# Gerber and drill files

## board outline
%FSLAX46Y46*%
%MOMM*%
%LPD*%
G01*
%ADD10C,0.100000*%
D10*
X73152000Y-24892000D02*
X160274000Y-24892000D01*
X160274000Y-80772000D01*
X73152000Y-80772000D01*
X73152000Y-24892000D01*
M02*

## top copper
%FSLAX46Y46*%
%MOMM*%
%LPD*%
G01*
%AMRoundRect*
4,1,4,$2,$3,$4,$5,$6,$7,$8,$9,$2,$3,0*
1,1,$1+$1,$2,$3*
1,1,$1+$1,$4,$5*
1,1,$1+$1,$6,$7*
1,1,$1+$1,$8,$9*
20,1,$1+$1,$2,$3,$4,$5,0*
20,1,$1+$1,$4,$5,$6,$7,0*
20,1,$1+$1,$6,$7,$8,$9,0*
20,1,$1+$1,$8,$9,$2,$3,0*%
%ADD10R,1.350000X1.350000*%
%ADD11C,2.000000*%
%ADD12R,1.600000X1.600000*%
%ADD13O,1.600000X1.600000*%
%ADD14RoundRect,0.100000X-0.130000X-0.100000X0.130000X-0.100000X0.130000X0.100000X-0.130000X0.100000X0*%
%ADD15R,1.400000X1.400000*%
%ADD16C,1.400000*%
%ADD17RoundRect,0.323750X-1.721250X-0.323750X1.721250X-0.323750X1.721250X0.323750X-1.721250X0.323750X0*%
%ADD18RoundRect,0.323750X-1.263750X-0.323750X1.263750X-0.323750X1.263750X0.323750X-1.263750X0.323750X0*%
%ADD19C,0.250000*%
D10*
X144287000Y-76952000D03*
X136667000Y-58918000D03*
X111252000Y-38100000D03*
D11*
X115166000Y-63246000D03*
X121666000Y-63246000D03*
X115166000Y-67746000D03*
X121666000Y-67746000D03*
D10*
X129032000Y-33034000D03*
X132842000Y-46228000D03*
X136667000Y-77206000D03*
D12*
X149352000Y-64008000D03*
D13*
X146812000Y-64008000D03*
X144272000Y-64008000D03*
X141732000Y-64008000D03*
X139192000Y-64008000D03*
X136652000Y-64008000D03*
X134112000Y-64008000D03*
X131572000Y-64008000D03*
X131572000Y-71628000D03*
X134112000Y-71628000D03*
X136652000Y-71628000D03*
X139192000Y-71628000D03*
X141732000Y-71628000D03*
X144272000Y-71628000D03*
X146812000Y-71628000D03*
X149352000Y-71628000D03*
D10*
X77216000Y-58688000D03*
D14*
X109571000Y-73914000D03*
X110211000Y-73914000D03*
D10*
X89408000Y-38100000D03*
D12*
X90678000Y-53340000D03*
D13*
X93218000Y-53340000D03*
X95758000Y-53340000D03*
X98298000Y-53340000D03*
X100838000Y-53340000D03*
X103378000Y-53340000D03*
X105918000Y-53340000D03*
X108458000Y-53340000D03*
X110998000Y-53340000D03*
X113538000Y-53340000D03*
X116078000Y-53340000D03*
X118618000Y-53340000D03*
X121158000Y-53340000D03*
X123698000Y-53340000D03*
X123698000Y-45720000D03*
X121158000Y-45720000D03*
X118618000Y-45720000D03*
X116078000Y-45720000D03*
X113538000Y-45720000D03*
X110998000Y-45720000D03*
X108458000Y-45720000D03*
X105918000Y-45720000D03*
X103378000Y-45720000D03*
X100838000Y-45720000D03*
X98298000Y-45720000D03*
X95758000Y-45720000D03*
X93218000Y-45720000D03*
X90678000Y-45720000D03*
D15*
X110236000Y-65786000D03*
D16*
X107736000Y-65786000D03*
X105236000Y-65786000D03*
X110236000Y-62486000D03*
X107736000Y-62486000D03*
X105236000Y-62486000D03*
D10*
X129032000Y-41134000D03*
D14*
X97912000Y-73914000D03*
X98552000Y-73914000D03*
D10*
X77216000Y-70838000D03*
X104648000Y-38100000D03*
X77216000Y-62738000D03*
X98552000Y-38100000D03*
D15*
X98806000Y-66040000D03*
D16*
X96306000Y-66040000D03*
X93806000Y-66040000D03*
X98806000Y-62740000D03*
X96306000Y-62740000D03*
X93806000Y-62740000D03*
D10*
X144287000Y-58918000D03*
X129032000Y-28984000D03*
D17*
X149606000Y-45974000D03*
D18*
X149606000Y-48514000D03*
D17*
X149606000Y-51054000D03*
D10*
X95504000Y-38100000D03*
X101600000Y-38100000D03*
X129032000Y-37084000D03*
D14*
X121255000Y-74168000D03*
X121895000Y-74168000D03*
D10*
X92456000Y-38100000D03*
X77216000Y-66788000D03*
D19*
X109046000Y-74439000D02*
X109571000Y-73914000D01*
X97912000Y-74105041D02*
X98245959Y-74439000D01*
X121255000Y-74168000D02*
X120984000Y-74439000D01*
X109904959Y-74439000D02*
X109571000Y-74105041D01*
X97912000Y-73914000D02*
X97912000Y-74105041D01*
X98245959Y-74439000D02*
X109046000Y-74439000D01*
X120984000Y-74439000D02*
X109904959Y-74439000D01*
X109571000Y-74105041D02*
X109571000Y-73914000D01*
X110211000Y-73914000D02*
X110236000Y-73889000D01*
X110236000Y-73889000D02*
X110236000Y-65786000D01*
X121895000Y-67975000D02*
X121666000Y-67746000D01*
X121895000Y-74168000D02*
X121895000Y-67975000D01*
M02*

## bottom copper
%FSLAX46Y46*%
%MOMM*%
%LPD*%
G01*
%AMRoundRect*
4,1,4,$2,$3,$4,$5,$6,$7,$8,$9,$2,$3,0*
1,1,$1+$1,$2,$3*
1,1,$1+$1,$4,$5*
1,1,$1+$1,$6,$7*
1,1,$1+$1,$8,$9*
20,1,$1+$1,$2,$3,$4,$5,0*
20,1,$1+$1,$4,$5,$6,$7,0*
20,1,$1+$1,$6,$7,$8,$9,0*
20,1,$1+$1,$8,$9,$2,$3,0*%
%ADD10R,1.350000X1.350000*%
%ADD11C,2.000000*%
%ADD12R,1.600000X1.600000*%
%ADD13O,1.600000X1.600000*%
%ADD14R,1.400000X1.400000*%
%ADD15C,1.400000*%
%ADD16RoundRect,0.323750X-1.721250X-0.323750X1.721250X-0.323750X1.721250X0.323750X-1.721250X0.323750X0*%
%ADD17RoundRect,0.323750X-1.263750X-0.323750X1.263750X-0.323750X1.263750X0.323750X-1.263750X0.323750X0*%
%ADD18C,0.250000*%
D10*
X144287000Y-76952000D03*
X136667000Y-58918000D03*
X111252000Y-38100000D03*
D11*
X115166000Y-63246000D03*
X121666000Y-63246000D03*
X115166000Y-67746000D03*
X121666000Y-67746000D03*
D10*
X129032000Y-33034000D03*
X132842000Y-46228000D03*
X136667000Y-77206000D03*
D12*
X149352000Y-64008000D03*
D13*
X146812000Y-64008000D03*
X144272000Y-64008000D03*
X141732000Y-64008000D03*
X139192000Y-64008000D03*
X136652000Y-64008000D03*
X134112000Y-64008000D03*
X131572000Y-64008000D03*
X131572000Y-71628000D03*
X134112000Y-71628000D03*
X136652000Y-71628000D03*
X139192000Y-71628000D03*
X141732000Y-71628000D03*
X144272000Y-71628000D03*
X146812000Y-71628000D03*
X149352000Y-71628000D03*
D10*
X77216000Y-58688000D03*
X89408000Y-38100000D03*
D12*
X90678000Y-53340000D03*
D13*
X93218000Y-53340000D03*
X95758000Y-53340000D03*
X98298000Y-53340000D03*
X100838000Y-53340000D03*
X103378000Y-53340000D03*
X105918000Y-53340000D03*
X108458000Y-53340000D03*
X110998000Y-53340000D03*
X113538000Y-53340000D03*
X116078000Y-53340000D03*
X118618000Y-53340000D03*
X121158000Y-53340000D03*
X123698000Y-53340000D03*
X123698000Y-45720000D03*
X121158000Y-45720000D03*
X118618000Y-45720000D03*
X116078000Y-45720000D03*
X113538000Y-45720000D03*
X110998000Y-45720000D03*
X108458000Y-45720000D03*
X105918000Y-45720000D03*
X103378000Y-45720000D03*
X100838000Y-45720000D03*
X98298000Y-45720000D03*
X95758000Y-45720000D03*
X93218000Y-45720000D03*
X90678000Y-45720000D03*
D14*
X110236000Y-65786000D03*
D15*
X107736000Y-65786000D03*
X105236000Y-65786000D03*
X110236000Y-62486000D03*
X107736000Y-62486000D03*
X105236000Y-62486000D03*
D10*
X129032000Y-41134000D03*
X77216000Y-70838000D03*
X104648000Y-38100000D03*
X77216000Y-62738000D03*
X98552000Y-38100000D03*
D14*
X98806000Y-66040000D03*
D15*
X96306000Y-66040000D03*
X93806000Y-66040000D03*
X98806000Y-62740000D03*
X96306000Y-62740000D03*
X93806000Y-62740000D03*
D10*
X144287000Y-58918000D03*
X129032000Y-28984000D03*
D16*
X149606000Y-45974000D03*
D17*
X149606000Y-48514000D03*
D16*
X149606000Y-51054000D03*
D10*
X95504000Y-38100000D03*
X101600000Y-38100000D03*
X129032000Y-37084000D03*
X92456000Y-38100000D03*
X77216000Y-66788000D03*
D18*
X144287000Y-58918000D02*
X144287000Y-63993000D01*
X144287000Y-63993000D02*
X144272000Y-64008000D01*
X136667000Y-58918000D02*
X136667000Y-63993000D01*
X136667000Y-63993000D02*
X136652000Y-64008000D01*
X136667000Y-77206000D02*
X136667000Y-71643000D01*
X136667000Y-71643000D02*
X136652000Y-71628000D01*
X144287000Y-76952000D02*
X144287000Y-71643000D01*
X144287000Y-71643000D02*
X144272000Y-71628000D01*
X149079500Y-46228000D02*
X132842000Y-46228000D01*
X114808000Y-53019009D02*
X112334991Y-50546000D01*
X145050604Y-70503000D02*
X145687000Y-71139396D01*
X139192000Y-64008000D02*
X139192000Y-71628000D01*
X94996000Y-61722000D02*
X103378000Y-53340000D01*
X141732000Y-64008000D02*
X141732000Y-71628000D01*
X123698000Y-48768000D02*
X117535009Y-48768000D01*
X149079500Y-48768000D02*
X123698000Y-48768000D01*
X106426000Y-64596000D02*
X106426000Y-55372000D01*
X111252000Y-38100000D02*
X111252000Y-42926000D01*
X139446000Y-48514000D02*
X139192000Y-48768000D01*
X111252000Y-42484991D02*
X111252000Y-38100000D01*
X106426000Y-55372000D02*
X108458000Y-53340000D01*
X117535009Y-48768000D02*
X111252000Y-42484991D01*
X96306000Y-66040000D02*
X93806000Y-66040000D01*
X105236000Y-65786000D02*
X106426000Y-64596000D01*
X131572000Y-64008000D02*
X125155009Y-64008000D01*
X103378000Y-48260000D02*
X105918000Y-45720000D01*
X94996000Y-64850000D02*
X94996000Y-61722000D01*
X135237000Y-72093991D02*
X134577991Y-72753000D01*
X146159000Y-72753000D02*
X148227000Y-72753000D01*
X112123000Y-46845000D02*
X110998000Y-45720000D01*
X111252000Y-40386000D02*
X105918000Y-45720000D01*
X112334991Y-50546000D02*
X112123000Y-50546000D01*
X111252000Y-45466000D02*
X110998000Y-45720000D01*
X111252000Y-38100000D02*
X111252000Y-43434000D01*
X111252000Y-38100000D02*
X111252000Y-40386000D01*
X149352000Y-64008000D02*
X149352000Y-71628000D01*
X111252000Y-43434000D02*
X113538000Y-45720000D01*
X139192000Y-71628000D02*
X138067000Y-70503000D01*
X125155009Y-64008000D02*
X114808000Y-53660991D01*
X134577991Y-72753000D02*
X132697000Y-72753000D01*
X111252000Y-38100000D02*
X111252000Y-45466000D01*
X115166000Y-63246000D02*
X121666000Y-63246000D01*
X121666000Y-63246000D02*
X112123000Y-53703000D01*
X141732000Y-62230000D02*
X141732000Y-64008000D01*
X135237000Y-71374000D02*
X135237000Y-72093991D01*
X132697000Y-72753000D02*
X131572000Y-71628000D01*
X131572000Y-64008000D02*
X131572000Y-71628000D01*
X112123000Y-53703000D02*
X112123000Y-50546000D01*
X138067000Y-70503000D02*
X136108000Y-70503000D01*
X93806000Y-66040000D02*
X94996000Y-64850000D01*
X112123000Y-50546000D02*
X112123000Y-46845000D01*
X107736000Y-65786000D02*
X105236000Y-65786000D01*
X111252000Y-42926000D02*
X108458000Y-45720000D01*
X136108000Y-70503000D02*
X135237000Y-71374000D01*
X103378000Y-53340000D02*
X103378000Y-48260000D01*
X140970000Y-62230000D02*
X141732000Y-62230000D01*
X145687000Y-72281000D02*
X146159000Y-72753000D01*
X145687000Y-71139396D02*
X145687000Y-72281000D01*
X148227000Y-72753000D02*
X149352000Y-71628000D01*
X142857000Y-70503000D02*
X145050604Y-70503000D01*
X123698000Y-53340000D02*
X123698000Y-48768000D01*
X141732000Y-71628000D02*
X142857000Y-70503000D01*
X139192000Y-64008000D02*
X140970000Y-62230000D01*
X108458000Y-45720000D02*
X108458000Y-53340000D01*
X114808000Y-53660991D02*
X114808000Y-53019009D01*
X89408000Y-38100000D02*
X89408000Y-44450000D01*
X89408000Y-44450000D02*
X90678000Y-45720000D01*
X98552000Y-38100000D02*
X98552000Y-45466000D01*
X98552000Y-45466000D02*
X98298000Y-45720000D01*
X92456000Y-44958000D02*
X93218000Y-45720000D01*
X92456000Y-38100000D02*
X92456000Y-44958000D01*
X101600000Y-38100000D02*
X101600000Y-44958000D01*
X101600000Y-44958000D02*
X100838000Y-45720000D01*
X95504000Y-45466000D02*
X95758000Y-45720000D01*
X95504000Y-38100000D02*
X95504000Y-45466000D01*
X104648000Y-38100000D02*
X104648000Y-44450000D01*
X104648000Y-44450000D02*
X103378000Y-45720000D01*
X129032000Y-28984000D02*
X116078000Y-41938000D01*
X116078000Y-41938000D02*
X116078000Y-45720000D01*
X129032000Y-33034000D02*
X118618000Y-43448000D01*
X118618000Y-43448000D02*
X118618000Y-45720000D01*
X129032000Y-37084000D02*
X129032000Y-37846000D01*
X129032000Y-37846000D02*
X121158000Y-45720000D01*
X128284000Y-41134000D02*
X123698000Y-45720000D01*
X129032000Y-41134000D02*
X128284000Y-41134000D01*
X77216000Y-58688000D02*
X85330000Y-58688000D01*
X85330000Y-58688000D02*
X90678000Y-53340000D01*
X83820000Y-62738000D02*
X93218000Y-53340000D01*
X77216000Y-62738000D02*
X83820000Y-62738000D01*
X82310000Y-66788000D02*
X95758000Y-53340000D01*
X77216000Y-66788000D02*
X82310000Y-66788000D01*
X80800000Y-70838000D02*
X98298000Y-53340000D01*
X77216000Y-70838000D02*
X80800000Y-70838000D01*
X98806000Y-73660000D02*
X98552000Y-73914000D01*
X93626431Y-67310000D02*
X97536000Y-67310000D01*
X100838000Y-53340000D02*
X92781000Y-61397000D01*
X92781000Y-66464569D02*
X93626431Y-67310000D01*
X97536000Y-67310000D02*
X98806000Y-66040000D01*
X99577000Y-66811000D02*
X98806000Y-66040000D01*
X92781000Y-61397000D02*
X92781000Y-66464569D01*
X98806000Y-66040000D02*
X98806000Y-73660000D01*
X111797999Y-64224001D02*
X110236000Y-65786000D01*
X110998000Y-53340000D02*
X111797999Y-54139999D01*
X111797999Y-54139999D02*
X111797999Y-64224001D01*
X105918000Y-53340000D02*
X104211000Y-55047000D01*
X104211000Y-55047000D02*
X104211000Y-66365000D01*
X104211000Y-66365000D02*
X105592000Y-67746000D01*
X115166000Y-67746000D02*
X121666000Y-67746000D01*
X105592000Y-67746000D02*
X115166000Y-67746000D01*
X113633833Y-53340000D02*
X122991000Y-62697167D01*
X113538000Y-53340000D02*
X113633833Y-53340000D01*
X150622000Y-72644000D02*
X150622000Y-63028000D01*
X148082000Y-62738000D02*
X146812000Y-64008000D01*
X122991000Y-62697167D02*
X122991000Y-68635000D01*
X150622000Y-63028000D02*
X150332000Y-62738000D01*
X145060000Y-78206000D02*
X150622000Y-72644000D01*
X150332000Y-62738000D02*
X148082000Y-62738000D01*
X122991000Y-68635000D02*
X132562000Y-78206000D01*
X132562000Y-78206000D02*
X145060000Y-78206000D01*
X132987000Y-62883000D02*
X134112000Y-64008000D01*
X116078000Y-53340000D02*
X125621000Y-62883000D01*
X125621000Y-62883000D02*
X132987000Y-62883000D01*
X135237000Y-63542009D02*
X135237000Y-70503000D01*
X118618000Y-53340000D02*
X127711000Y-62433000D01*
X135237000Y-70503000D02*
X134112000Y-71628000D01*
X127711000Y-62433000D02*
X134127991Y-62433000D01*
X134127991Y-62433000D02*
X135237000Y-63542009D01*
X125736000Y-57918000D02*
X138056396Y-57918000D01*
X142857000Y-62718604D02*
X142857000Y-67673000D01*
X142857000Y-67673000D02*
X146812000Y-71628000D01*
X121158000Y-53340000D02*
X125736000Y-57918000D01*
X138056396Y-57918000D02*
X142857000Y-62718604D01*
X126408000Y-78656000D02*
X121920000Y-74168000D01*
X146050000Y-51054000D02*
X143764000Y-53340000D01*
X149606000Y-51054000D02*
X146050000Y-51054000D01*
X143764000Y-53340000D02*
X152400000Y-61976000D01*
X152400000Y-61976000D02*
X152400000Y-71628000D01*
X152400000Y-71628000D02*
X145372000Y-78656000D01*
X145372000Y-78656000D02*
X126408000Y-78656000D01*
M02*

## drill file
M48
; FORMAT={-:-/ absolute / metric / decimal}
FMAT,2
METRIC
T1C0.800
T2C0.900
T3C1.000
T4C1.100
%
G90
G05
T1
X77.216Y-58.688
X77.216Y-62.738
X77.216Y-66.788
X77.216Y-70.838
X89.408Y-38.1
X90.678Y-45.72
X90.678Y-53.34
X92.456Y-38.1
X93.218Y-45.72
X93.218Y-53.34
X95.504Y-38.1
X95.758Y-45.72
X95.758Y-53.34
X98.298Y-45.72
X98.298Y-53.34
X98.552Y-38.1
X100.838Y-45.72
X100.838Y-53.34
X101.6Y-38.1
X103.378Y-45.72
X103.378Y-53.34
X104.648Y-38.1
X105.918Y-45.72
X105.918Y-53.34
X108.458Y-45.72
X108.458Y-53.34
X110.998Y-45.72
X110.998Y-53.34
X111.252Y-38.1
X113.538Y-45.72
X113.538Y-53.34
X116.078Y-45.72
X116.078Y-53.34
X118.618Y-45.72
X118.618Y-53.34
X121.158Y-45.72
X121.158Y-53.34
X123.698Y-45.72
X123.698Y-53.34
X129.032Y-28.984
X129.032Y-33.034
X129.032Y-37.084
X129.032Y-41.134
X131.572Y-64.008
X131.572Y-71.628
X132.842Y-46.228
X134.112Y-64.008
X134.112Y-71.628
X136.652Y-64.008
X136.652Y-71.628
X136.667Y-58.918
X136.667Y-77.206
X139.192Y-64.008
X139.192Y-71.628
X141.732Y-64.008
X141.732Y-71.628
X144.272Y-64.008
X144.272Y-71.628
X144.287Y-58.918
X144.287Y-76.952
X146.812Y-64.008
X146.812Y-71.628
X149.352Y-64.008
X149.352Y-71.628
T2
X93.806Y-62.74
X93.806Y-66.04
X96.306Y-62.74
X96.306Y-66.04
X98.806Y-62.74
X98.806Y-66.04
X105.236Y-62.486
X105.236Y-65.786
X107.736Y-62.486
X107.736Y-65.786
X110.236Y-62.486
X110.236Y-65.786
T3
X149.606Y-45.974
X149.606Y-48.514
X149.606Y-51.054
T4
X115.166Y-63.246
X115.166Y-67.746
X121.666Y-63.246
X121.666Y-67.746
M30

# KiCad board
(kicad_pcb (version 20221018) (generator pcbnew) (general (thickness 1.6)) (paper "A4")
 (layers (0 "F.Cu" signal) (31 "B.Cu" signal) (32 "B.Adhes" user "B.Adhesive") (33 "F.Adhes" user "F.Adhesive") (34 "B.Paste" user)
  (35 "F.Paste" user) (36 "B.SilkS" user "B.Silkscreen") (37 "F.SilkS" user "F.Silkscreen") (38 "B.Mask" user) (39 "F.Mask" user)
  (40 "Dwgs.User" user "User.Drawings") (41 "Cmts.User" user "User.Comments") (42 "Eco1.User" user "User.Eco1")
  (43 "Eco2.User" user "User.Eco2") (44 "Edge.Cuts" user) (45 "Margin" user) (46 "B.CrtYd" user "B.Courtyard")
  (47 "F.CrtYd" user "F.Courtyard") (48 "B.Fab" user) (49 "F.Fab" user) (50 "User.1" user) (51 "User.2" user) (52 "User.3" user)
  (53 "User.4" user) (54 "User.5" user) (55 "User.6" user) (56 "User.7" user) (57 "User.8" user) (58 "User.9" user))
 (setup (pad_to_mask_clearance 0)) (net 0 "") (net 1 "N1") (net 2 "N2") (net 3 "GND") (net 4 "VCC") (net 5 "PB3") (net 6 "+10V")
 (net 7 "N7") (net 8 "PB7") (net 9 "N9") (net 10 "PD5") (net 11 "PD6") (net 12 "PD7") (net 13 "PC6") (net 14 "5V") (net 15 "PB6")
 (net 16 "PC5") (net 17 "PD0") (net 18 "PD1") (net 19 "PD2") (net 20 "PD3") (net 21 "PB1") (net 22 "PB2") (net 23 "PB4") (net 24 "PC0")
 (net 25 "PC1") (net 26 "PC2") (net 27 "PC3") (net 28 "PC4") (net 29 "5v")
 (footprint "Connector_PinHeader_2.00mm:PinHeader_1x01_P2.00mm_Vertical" (layer "F.Cu") (at 144.287 76.952)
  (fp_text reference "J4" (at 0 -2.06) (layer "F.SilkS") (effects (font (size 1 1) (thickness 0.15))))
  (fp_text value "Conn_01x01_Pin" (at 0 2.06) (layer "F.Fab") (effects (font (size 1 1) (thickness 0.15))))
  (pad "1" thru_hole rect (at 0 0) (size 1.35 1.35) (drill 0.8) (layers "*.Cu" "*.Mask") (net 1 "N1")))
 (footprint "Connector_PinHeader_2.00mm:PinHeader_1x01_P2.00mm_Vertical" (layer "F.Cu") (at 136.667 58.918)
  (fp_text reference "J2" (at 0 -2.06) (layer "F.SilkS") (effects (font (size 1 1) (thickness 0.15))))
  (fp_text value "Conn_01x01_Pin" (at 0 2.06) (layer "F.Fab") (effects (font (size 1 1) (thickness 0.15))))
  (pad "1" thru_hole rect (at 0 0) (size 1.35 1.35) (drill 0.8) (layers "*.Cu" "*.Mask") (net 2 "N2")))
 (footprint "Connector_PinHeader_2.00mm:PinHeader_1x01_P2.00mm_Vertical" (layer "F.Cu") (at 111.252 38.1)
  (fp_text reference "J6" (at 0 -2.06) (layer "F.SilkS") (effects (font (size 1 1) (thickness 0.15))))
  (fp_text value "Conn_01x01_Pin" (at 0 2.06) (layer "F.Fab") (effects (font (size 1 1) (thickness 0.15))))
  (pad "1" thru_hole rect (at 0 0) (size 1.35 1.35) (drill 0.8) (layers "*.Cu" "*.Mask") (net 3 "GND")))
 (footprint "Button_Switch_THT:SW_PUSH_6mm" (layer "F.Cu") (at 115.166 63.246)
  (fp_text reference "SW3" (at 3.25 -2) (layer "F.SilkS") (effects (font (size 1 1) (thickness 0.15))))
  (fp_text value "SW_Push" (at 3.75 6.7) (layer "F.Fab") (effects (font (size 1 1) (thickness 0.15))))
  (pad "1" thru_hole circle (at 0 0 90) (size 2 2) (drill 1.1) (layers "*.Cu" "*.Mask") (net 3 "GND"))
  (pad "1" thru_hole circle (at 6.5 0 90) (size 2 2) (drill 1.1) (layers "*.Cu" "*.Mask") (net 3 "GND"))
  (pad "2" thru_hole circle (at 0 4.5 90) (size 2 2) (drill 1.1) (layers "*.Cu" "*.Mask") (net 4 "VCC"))
  (pad "2" thru_hole circle (at 6.5 4.5 90) (size 2 2) (drill 1.1) (layers "*.Cu" "*.Mask") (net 4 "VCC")))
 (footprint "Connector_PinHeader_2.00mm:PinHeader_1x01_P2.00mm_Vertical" (layer "F.Cu") (at 129.032 33.034)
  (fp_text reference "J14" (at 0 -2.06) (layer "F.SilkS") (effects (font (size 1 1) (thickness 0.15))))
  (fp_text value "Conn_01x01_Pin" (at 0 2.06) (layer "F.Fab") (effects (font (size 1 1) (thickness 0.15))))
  (pad "1" thru_hole rect (at 0 0) (size 1.35 1.35) (drill 0.8) (layers "*.Cu" "*.Mask") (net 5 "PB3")))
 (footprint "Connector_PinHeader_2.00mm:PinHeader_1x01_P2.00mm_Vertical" (layer "F.Cu") (at 132.842 46.228)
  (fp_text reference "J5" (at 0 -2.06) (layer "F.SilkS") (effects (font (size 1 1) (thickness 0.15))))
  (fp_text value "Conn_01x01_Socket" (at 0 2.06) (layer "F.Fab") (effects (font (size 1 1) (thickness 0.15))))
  (pad "1" thru_hole rect (at 0 0) (size 1.35 1.35) (drill 0.8) (layers "*.Cu" "*.Mask") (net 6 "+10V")))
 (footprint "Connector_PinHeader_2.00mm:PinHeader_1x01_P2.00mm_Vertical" (layer "F.Cu") (at 136.667 77.206)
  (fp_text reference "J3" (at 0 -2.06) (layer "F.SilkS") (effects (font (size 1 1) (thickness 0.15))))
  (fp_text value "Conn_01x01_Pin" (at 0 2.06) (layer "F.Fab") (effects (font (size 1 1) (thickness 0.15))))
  (pad "1" thru_hole rect (at 0 0) (size 1.35 1.35) (drill 0.8) (layers "*.Cu" "*.Mask") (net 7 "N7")))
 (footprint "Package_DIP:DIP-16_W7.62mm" (layer "F.Cu") (at 149.352 64.008 -90)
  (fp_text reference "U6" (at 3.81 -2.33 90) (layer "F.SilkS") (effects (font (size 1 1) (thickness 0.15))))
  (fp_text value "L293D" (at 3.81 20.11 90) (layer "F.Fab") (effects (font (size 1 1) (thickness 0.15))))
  (pad "1" thru_hole rect (at 0 0 270) (size 1.6 1.6) (drill 0.8) (layers "*.Cu" "*.Mask") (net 3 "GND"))
  (pad "2" thru_hole oval (at 0 2.54 270) (size 1.6 1.6) (drill 0.8) (layers "*.Cu" "*.Mask") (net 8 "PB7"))
  (pad "3" thru_hole oval (at 0 5.08 270) (size 1.6 1.6) (drill 0.8) (layers "*.Cu" "*.Mask") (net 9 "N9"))
  (pad "4" thru_hole oval (at 0 7.62 270) (size 1.6 1.6) (drill 0.8) (layers "*.Cu" "*.Mask") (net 3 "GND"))
  (pad "5" thru_hole oval (at 0 10.16 270) (size 1.6 1.6) (drill 0.8) (layers "*.Cu" "*.Mask") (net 3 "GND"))
  (pad "6" thru_hole oval (at 0 12.7 270) (size 1.6 1.6) (drill 0.8) (layers "*.Cu" "*.Mask") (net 2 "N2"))
  (pad "7" thru_hole oval (at 0 15.24 270) (size 1.6 1.6) (drill 0.8) (layers "*.Cu" "*.Mask") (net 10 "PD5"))
  (pad "8" thru_hole oval (at 0 17.78 270) (size 1.6 1.6) (drill 0.8) (layers "*.Cu" "*.Mask") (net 3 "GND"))
  (pad "9" thru_hole oval (at 7.62 17.78 270) (size 1.6 1.6) (drill 0.8) (layers "*.Cu" "*.Mask") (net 3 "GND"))
  (pad "10" thru_hole oval (at 7.62 15.24 270) (size 1.6 1.6) (drill 0.8) (layers "*.Cu" "*.Mask") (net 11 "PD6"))
  (pad "11" thru_hole oval (at 7.62 12.7 270) (size 1.6 1.6) (drill 0.8) (layers "*.Cu" "*.Mask") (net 7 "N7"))
  (pad "12" thru_hole oval (at 7.62 10.16 270) (size 1.6 1.6) (drill 0.8) (layers "*.Cu" "*.Mask") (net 3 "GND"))
  (pad "13" thru_hole oval (at 7.62 7.62 270) (size 1.6 1.6) (drill 0.8) (layers "*.Cu" "*.Mask") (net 3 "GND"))
  (pad "14" thru_hole oval (at 7.62 5.08 270) (size 1.6 1.6) (drill 0.8) (layers "*.Cu" "*.Mask") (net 1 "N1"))
  (pad "15" thru_hole oval (at 7.62 2.54 270) (size 1.6 1.6) (drill 0.8) (layers "*.Cu" "*.Mask") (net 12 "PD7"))
  (pad "16" thru_hole oval (at 7.62 0 270) (size 1.6 1.6) (drill 0.8) (layers "*.Cu" "*.Mask") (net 3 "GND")))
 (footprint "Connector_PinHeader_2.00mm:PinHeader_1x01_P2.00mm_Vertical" (layer "F.Cu") (at 77.216 58.688)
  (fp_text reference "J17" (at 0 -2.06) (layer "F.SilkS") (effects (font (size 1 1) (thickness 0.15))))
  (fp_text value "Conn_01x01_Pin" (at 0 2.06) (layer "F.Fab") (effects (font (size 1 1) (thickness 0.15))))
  (pad "1" thru_hole rect (at 0 0) (size 1.35 1.35) (drill 0.8) (layers "*.Cu" "*.Mask") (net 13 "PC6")))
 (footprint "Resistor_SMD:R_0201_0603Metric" (layer "F.Cu") (at 109.891 73.914)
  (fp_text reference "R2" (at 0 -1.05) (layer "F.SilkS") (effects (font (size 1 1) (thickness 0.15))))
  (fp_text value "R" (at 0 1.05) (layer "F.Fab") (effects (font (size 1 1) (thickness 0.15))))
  (pad "" smd roundrect (at -0.345 0) (size 0.318 0.36) (layers "F.Paste") (roundrect_rratio 0.25))
  (pad "" smd roundrect (at 0.345 0) (size 0.318 0.36) (layers "F.Paste") (roundrect_rratio 0.25))
  (pad "1" smd roundrect (at -0.32 0) (size 0.46 0.4) (layers "F.Cu" "F.Mask") (roundrect_rratio 0.25) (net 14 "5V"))
  (pad "2" smd roundrect (at 0.32 0) (size 0.46 0.4) (layers "F.Cu" "F.Mask") (roundrect_rratio 0.25) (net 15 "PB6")))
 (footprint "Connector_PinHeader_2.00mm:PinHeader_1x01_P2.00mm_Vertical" (layer "F.Cu") (at 89.408 38.1)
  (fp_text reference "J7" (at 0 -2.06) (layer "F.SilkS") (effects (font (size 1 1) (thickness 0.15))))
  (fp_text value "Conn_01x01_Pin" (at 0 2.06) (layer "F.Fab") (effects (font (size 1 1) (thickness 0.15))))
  (pad "1" thru_hole rect (at 0 0) (size 1.35 1.35) (drill 0.8) (layers "*.Cu" "*.Mask") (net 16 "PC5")))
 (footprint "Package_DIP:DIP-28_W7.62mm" (layer "F.Cu") (at 90.678 53.34 90)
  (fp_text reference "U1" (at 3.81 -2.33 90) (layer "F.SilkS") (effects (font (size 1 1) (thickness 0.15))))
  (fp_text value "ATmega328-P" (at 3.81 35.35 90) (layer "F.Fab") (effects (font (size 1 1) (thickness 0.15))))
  (pad "1" thru_hole rect (at 0 0 90) (size 1.6 1.6) (drill 0.8) (layers "*.Cu" "*.Mask") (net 13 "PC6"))
  (pad "2" thru_hole oval (at 0 2.54 90) (size 1.6 1.6) (drill 0.8) (layers "*.Cu" "*.Mask") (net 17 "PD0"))
  (pad "3" thru_hole oval (at 0 5.08 90) (size 1.6 1.6) (drill 0.8) (layers "*.Cu" "*.Mask") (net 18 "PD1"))
  (pad "4" thru_hole oval (at 0 7.62 90) (size 1.6 1.6) (drill 0.8) (layers "*.Cu" "*.Mask") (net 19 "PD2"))
  (pad "5" thru_hole oval (at 0 10.16 90) (size 1.6 1.6) (drill 0.8) (layers "*.Cu" "*.Mask") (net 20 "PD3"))
  (pad "6" thru_hole oval (at 0 12.7 90) (size 1.6 1.6) (drill 0.8) (layers "*.Cu" "*.Mask") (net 3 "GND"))
  (pad "7" thru_hole oval (at 0 15.24 90) (size 1.6 1.6) (drill 0.8) (layers "*.Cu" "*.Mask") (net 4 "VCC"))
  (pad "8" thru_hole oval (at 0 17.78 90) (size 1.6 1.6) (drill 0.8) (layers "*.Cu" "*.Mask") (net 3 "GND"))
  (pad "9" thru_hole oval (at 0 20.32 90) (size 1.6 1.6) (drill 0.8) (layers "*.Cu" "*.Mask") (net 15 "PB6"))
  (pad "10" thru_hole oval (at 0 22.86 90) (size 1.6 1.6) (drill 0.8) (layers "*.Cu" "*.Mask") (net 8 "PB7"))
  (pad "11" thru_hole oval (at 0 25.4 90) (size 1.6 1.6) (drill 0.8) (layers "*.Cu" "*.Mask") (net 10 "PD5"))
  (pad "12" thru_hole oval (at 0 27.94 90) (size 1.6 1.6) (drill 0.8) (layers "*.Cu" "*.Mask") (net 11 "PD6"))
  (pad "13" thru_hole oval (at 0 30.48 90) (size 1.6 1.6) (drill 0.8) (layers "*.Cu" "*.Mask") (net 12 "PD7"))
  (pad "14" thru_hole oval (at 0 33.02 90) (size 1.6 1.6) (drill 0.8) (layers "*.Cu" "*.Mask") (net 3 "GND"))
  (pad "15" thru_hole oval (at 7.62 33.02 90) (size 1.6 1.6) (drill 0.8) (layers "*.Cu" "*.Mask") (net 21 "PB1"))
  (pad "16" thru_hole oval (at 7.62 30.48 90) (size 1.6 1.6) (drill 0.8) (layers "*.Cu" "*.Mask") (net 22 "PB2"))
  (pad "17" thru_hole oval (at 7.62 27.94 90) (size 1.6 1.6) (drill 0.8) (layers "*.Cu" "*.Mask") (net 5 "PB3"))
  (pad "18" thru_hole oval (at 7.62 25.4 90) (size 1.6 1.6) (drill 0.8) (layers "*.Cu" "*.Mask") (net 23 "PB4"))
  (pad "19" thru_hole oval (at 7.62 22.86 90) (size 1.6 1.6) (drill 0.8) (layers "*.Cu" "*.Mask") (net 3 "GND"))
  (pad "20" thru_hole oval (at 7.62 20.32 90) (size 1.6 1.6) (drill 0.8) (layers "*.Cu" "*.Mask") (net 3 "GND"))
  (pad "21" thru_hole oval (at 7.62 17.78 90) (size 1.6 1.6) (drill 0.8) (layers "*.Cu" "*.Mask") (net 3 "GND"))
  (pad "22" thru_hole oval (at 7.62 15.24 90) (size 1.6 1.6) (drill 0.8) (layers "*.Cu" "*.Mask") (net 3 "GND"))
  (pad "23" thru_hole oval (at 7.62 12.7 90) (size 1.6 1.6) (drill 0.8) (layers "*.Cu" "*.Mask") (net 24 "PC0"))
  (pad "24" thru_hole oval (at 7.62 10.16 90) (size 1.6 1.6) (drill 0.8) (layers "*.Cu" "*.Mask") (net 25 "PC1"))
  (pad "25" thru_hole oval (at 7.62 7.62 90) (size 1.6 1.6) (drill 0.8) (layers "*.Cu" "*.Mask") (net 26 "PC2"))
  (pad "26" thru_hole oval (at 7.62 5.08 90) (size 1.6 1.6) (drill 0.8) (layers "*.Cu" "*.Mask") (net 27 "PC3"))
  (pad "27" thru_hole oval (at 7.62 2.54 90) (size 1.6 1.6) (drill 0.8) (layers "*.Cu" "*.Mask") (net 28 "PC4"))
  (pad "28" thru_hole oval (at 7.62 0 90) (size 1.6 1.6) (drill 0.8) (layers "*.Cu" "*.Mask") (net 16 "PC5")))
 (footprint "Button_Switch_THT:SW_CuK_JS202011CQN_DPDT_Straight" (layer "F.Cu") (at 110.236 65.786 180)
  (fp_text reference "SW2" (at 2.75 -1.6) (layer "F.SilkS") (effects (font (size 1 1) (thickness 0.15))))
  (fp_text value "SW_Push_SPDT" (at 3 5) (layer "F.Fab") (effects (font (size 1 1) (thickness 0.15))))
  (pad "1" thru_hole rect (at 0 0 180) (size 1.4 1.4) (drill 0.9) (layers "*.Cu" "*.Mask") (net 15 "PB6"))
  (pad "2" thru_hole circle (at 2.5 0 180) (size 1.4 1.4) (drill 0.9) (layers "*.Cu" "*.Mask") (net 3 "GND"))
  (pad "3" thru_hole circle (at 5 0 180) (size 1.4 1.4) (drill 0.9) (layers "*.Cu" "*.Mask") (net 3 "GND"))
  (pad "4" thru_hole circle (at 0 3.3 180) (size 1.4 1.4) (drill 0.9) (layers "*.Cu" "*.Mask"))
  (pad "5" thru_hole circle (at 2.5 3.3 180) (size 1.4 1.4) (drill 0.9) (layers "*.Cu" "*.Mask"))
  (pad "6" thru_hole circle (at 5 3.3 180) (size 1.4 1.4) (drill 0.9) (layers "*.Cu" "*.Mask")))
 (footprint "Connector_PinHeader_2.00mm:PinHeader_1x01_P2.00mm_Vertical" (layer "F.Cu") (at 129.032 41.134)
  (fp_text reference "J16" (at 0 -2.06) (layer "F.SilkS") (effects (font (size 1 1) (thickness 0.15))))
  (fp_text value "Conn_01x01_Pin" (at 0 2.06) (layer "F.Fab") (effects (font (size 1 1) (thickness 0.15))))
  (pad "1" thru_hole rect (at 0 0) (size 1.35 1.35) (drill 0.8) (layers "*.Cu" "*.Mask") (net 21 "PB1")))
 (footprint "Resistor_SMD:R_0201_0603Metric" (layer "F.Cu") (at 98.232 73.914)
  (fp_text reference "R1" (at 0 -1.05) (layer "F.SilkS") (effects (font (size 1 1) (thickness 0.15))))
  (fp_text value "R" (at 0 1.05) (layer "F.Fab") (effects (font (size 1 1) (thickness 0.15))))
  (pad "" smd roundrect (at -0.345 0) (size 0.318 0.36) (layers "F.Paste") (roundrect_rratio 0.25))
  (pad "" smd roundrect (at 0.345 0) (size 0.318 0.36) (layers "F.Paste") (roundrect_rratio 0.25))
  (pad "1" smd roundrect (at -0.32 0) (size 0.46 0.4) (layers "F.Cu" "F.Mask") (roundrect_rratio 0.25) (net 14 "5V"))
  (pad "2" smd roundrect (at 0.32 0) (size 0.46 0.4) (layers "F.Cu" "F.Mask") (roundrect_rratio 0.25) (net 20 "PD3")))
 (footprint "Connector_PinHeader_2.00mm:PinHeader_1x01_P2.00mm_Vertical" (layer "F.Cu") (at 77.216 70.838)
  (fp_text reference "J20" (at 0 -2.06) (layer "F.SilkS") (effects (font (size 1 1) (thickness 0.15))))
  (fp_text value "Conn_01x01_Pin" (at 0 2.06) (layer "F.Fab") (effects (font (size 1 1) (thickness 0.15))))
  (pad "1" thru_hole rect (at 0 0) (size 1.35 1.35) (drill 0.8) (layers "*.Cu" "*.Mask") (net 19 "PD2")))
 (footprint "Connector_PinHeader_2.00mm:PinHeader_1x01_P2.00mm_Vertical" (layer "F.Cu") (at 104.648 38.1)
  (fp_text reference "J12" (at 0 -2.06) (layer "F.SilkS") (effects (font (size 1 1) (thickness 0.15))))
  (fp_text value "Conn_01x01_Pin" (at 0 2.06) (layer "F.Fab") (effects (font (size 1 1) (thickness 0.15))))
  (pad "1" thru_hole rect (at 0 0) (size 1.35 1.35) (drill 0.8) (layers "*.Cu" "*.Mask") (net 24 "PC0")))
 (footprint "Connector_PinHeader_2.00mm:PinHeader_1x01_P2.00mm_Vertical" (layer "F.Cu") (at 77.216 62.738)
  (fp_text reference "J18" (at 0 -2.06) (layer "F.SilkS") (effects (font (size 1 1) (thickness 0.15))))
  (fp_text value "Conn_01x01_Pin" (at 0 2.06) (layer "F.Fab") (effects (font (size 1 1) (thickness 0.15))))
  (pad "1" thru_hole rect (at 0 0) (size 1.35 1.35) (drill 0.8) (layers "*.Cu" "*.Mask") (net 17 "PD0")))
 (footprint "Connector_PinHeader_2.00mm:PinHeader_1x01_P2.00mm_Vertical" (layer "F.Cu") (at 98.552 38.1)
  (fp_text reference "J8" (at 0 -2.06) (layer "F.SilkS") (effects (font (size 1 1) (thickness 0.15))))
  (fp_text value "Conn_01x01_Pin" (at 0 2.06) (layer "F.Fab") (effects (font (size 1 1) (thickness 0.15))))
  (pad "1" thru_hole rect (at 0 0) (size 1.35 1.35) (drill 0.8) (layers "*.Cu" "*.Mask") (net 26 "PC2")))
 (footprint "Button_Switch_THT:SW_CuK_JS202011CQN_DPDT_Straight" (layer "F.Cu") (at 98.806 66.04 180)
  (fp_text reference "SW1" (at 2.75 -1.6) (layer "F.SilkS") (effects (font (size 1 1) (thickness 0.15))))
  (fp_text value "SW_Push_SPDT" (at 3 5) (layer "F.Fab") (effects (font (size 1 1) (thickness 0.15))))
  (pad "1" thru_hole rect (at 0 0 180) (size 1.4 1.4) (drill 0.9) (layers "*.Cu" "*.Mask") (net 20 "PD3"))
  (pad "2" thru_hole circle (at 2.5 0 180) (size 1.4 1.4) (drill 0.9) (layers "*.Cu" "*.Mask") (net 3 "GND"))
  (pad "3" thru_hole circle (at 5 0 180) (size 1.4 1.4) (drill 0.9) (layers "*.Cu" "*.Mask") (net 3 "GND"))
  (pad "4" thru_hole circle (at 0 3.3 180) (size 1.4 1.4) (drill 0.9) (layers "*.Cu" "*.Mask"))
  (pad "5" thru_hole circle (at 2.5 3.3 180) (size 1.4 1.4) (drill 0.9) (layers "*.Cu" "*.Mask"))
  (pad "6" thru_hole circle (at 5 3.3 180) (size 1.4 1.4) (drill 0.9) (layers "*.Cu" "*.Mask")))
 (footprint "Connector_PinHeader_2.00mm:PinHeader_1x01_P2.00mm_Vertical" (layer "F.Cu") (at 144.287 58.918)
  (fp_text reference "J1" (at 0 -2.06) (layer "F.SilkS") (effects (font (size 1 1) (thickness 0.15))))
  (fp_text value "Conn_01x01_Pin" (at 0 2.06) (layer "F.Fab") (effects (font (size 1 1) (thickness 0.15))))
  (pad "1" thru_hole rect (at 0 0) (size 1.35 1.35) (drill 0.8) (layers "*.Cu" "*.Mask") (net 9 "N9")))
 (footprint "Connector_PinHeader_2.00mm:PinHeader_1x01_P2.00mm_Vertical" (layer "F.Cu") (at 129.032 28.984)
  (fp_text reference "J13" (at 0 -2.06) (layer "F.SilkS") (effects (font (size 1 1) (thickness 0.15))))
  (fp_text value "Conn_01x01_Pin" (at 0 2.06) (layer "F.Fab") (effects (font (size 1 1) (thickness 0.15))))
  (pad "1" thru_hole rect (at 0 0) (size 1.35 1.35) (drill 0.8) (layers "*.Cu" "*.Mask") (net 23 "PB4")))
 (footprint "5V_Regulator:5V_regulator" (layer "F.Cu") (at 154.686 45.974)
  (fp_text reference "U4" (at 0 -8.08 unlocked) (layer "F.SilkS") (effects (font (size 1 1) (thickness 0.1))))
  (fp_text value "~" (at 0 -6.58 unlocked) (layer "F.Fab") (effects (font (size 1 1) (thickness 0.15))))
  (pad "1" thru_hole roundrect (at -5.08 0) (size 4.09 1.295) (drill 1) (layers "*.Cu" "*.Mask") (roundrect_rratio 0.25) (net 6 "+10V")
   (thermal_bridge_angle 45))
  (pad "2" thru_hole roundrect (at -5.08 2.54) (size 3.175 1.295) (drill 1) (layers "*.Cu" "*.Mask") (roundrect_rratio 0.25) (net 3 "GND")
   (thermal_bridge_angle 45))
  (pad "3" thru_hole roundrect (at -5.08 5.08) (size 4.09 1.295) (drill 1) (layers "*.Cu" "*.Mask") (roundrect_rratio 0.25) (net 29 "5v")
   (thermal_bridge_angle 45)))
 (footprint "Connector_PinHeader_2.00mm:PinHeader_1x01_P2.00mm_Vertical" (layer "F.Cu") (at 95.504 38.1)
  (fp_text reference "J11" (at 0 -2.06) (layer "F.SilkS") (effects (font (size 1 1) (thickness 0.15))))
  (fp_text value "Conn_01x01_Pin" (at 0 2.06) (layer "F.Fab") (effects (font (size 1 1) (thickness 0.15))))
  (pad "1" thru_hole rect (at 0 0) (size 1.35 1.35) (drill 0.8) (layers "*.Cu" "*.Mask") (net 27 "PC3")))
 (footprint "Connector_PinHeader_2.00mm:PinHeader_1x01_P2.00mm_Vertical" (layer "F.Cu") (at 101.6 38.1)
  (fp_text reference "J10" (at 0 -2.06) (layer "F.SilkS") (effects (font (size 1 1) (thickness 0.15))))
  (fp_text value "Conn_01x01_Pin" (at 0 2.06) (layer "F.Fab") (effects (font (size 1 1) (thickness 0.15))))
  (pad "1" thru_hole rect (at 0 0) (size 1.35 1.35) (drill 0.8) (layers "*.Cu" "*.Mask") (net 25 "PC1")))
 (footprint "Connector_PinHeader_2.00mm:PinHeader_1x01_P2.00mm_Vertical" (layer "F.Cu") (at 129.032 37.084)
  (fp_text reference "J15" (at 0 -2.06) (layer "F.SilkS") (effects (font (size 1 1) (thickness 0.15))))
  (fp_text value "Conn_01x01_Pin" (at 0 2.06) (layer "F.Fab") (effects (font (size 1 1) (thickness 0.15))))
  (pad "1" thru_hole rect (at 0 0) (size 1.35 1.35) (drill 0.8) (layers "*.Cu" "*.Mask") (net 22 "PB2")))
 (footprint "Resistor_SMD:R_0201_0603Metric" (layer "F.Cu") (at 121.575 74.168)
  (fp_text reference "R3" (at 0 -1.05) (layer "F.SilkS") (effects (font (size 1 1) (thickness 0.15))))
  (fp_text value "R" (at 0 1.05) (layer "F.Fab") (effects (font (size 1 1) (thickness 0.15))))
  (pad "" smd roundrect (at -0.345 0) (size 0.318 0.36) (layers "F.Paste") (roundrect_rratio 0.25))
  (pad "" smd roundrect (at 0.345 0) (size 0.318 0.36) (layers "F.Paste") (roundrect_rratio 0.25))
  (pad "1" smd roundrect (at -0.32 0) (size 0.46 0.4) (layers "F.Cu" "F.Mask") (roundrect_rratio 0.25) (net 14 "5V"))
  (pad "2" smd roundrect (at 0.32 0) (size 0.46 0.4) (layers "F.Cu" "F.Mask") (roundrect_rratio 0.25) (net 4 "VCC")))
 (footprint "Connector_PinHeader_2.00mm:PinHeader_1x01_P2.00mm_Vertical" (layer "F.Cu") (at 92.456 38.1)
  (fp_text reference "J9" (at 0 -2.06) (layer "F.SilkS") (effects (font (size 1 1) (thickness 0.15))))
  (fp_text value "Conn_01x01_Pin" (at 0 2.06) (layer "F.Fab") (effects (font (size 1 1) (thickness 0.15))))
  (pad "1" thru_hole rect (at 0 0) (size 1.35 1.35) (drill 0.8) (layers "*.Cu" "*.Mask") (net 28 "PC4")))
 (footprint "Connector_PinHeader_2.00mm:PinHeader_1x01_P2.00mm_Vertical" (layer "F.Cu") (at 77.216 66.788)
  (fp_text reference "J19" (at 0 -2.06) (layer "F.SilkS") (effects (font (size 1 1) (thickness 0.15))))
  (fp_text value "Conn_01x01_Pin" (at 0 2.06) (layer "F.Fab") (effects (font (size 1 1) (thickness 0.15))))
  (pad "1" thru_hole rect (at 0 0) (size 1.35 1.35) (drill 0.8) (layers "*.Cu" "*.Mask") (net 18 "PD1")))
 (gr_rect (start 73.152 24.892) (end 160.274 80.772) (stroke (width 0.1) (type default)) (fill none) (layer "Edge.Cuts"))
 (segment (start 144.287 58.918) (end 144.287 63.993) (width 0.25) (layer "B.Cu") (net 9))
 (segment (start 144.287 63.993) (end 144.272 64.008) (width 0.25) (layer "B.Cu") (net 9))
 (segment (start 136.667 58.918) (end 136.667 63.993) (width 0.25) (layer "B.Cu") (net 2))
 (segment (start 136.667 63.993) (end 136.652 64.008) (width 0.25) (layer "B.Cu") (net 2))
 (segment (start 136.667 77.206) (end 136.667 71.643) (width 0.25) (layer "B.Cu") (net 7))
 (segment (start 136.667 71.643) (end 136.652 71.628) (width 0.25) (layer "B.Cu") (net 7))
 (segment (start 144.287 76.952) (end 144.287 71.643) (width 0.25) (layer "B.Cu") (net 1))
 (segment (start 144.287 71.643) (end 144.272 71.628) (width 0.25) (layer "B.Cu") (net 1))
 (segment (start 149.0795 46.228) (end 132.842 46.228) (width 0.25) (layer "B.Cu") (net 6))
 (segment (start 114.808 53.019009) (end 112.334991 50.546) (width 0.25) (layer "B.Cu") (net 3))
 (segment (start 145.050604 70.503) (end 145.687 71.139396) (width 0.25) (layer "B.Cu") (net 3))
 (segment (start 139.192 64.008) (end 139.192 71.628) (width 0.25) (layer "B.Cu") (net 3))
 (segment (start 94.996 61.722) (end 103.378 53.34) (width 0.25) (layer "B.Cu") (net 3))
 (segment (start 141.732 64.008) (end 141.732 71.628) (width 0.25) (layer "B.Cu") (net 3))
 (segment (start 123.698 48.768) (end 117.535009 48.768) (width 0.25) (layer "B.Cu") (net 3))
 (segment (start 149.0795 48.768) (end 123.698 48.768) (width 0.25) (layer "B.Cu") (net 3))
 (segment (start 106.426 64.596) (end 106.426 55.372) (width 0.25) (layer "B.Cu") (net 3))
 (segment (start 111.252 38.1) (end 111.252 42.926) (width 0.25) (layer "B.Cu") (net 3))
 (segment (start 139.446 48.514) (end 139.192 48.768) (width 0.25) (layer "B.Cu") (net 3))
 (segment (start 111.252 42.484991) (end 111.252 38.1) (width 0.25) (layer "B.Cu") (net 3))
 (segment (start 106.426 55.372) (end 108.458 53.34) (width 0.25) (layer "B.Cu") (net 3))
 (segment (start 117.535009 48.768) (end 111.252 42.484991) (width 0.25) (layer "B.Cu") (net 3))
 (segment (start 96.306 66.04) (end 93.806 66.04) (width 0.25) (layer "B.Cu") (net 3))
 (segment (start 105.236 65.786) (end 106.426 64.596) (width 0.25) (layer "B.Cu") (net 3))
 (segment (start 131.572 64.008) (end 125.155009 64.008) (width 0.25) (layer "B.Cu") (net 3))
 (segment (start 103.378 48.26) (end 105.918 45.72) (width 0.25) (layer "B.Cu") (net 3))
 (segment (start 94.996 64.85) (end 94.996 61.722) (width 0.25) (layer "B.Cu") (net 3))
 (segment (start 135.237 72.093991) (end 134.577991 72.753) (width 0.25) (layer "B.Cu") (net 3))
 (segment (start 146.159 72.753) (end 148.227 72.753) (width 0.25) (layer "B.Cu") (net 3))
 (segment (start 112.123 46.845) (end 110.998 45.72) (width 0.25) (layer "B.Cu") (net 3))
 (segment (start 111.252 40.386) (end 105.918 45.72) (width 0.25) (layer "B.Cu") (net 3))
 (segment (start 112.334991 50.546) (end 112.123 50.546) (width 0.25) (layer "B.Cu") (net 3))
 (segment (start 111.252 45.466) (end 110.998 45.72) (width 0.25) (layer "B.Cu") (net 3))
 (segment (start 111.252 38.1) (end 111.252 43.434) (width 0.25) (layer "B.Cu") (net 3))
 (segment (start 111.252 38.1) (end 111.252 40.386) (width 0.25) (layer "B.Cu") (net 3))
 (segment (start 149.352 64.008) (end 149.352 71.628) (width 0.25) (layer "B.Cu") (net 3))
 (segment (start 111.252 43.434) (end 113.538 45.72) (width 0.25) (layer "B.Cu") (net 3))
 (segment (start 139.192 71.628) (end 138.067 70.503) (width 0.25) (layer "B.Cu") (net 3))
 (segment (start 125.155009 64.008) (end 114.808 53.660991) (width 0.25) (layer "B.Cu") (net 3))
 (segment (start 134.577991 72.753) (end 132.697 72.753) (width 0.25) (layer "B.Cu") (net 3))
 (segment (start 111.252 38.1) (end 111.252 45.466) (width 0.25) (layer "B.Cu") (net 3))
 (segment (start 115.166 63.246) (end 121.666 63.246) (width 0.25) (layer "B.Cu") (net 3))
 (segment (start 121.666 63.246) (end 112.123 53.703) (width 0.25) (layer "B.Cu") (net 3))
 (segment (start 141.732 62.23) (end 141.732 64.008) (width 0.25) (layer "B.Cu") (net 3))
 (segment (start 135.237 71.374) (end 135.237 72.093991) (width 0.25) (layer "B.Cu") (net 3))
 (segment (start 132.697 72.753) (end 131.572 71.628) (width 0.25) (layer "B.Cu") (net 3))
 (segment (start 131.572 64.008) (end 131.572 71.628) (width 0.25) (layer "B.Cu") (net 3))
 (segment (start 112.123 53.703) (end 112.123 50.546) (width 0.25) (layer "B.Cu") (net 3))
 (segment (start 138.067 70.503) (end 136.108 70.503) (width 0.25) (layer "B.Cu") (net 3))
 (segment (start 93.806 66.04) (end 94.996 64.85) (width 0.25) (layer "B.Cu") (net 3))
 (segment (start 112.123 50.546) (end 112.123 46.845) (width 0.25) (layer "B.Cu") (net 3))
 (segment (start 107.736 65.786) (end 105.236 65.786) (width 0.25) (layer "B.Cu") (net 3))
 (segment (start 111.252 42.926) (end 108.458 45.72) (width 0.25) (layer "B.Cu") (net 3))
 (segment (start 136.108 70.503) (end 135.237 71.374) (width 0.25) (layer "B.Cu") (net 3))
 (segment (start 103.378 53.34) (end 103.378 48.26) (width 0.25) (layer "B.Cu") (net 3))
 (segment (start 140.97 62.23) (end 141.732 62.23) (width 0.25) (layer "B.Cu") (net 3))
 (segment (start 145.687 72.281) (end 146.159 72.753) (width 0.25) (layer "B.Cu") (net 3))
 (segment (start 145.687 71.139396) (end 145.687 72.281) (width 0.25) (layer "B.Cu") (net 3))
 (segment (start 148.227 72.753) (end 149.352 71.628) (width 0.25) (layer "B.Cu") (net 3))
 (segment (start 142.857 70.503) (end 145.050604 70.503) (width 0.25) (layer "B.Cu") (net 3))
 (segment (start 123.698 53.34) (end 123.698 48.768) (width 0.25) (layer "B.Cu") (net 3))
 (segment (start 141.732 71.628) (end 142.857 70.503) (width 0.25) (layer "B.Cu") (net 3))
 (segment (start 139.192 64.008) (end 140.97 62.23) (width 0.25) (layer "B.Cu") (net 3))
 (segment (start 108.458 45.72) (end 108.458 53.34) (width 0.25) (layer "B.Cu") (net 3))
 (segment (start 114.808 53.660991) (end 114.808 53.019009) (width 0.25) (layer "B.Cu") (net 3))
 (segment (start 89.408 38.1) (end 89.408 44.45) (width 0.25) (layer "B.Cu") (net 16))
 (segment (start 89.408 44.45) (end 90.678 45.72) (width 0.25) (layer "B.Cu") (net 16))
 (segment (start 98.552 38.1) (end 98.552 45.466) (width 0.25) (layer "B.Cu") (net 26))
 (segment (start 98.552 45.466) (end 98.298 45.72) (width 0.25) (layer "B.Cu") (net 26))
 (segment (start 92.456 44.958) (end 93.218 45.72) (width 0.25) (layer "B.Cu") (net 28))
 (segment (start 92.456 38.1) (end 92.456 44.958) (width 0.25) (layer "B.Cu") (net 28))
 (segment (start 101.6 38.1) (end 101.6 44.958) (width 0.25) (layer "B.Cu") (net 25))
 (segment (start 101.6 44.958) (end 100.838 45.72) (width 0.25) (layer "B.Cu") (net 25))
 (segment (start 95.504 45.466) (end 95.758 45.72) (width 0.25) (layer "B.Cu") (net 27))
 (segment (start 95.504 38.1) (end 95.504 45.466) (width 0.25) (layer "B.Cu") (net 27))
 (segment (start 104.648 38.1) (end 104.648 44.45) (width 0.25) (layer "B.Cu") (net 24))
 (segment (start 104.648 44.45) (end 103.378 45.72) (width 0.25) (layer "B.Cu") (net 24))
 (segment (start 129.032 28.984) (end 116.078 41.938) (width 0.25) (layer "B.Cu") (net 23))
 (segment (start 116.078 41.938) (end 116.078 45.72) (width 0.25) (layer "B.Cu") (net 23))
 (segment (start 129.032 33.034) (end 118.618 43.448) (width 0.25) (layer "B.Cu") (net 5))
 (segment (start 118.618 43.448) (end 118.618 45.72) (width 0.25) (layer "B.Cu") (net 5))
 (segment (start 129.032 37.084) (end 129.032 37.846) (width 0.25) (layer "B.Cu") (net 22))
 (segment (start 129.032 37.846) (end 121.158 45.72) (width 0.25) (layer "B.Cu") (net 22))
 (segment (start 128.284 41.134) (end 123.698 45.72) (width 0.25) (layer "B.Cu") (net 21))
 (segment (start 129.032 41.134) (end 128.284 41.134) (width 0.25) (layer "B.Cu") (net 21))
 (segment (start 77.216 58.688) (end 85.33 58.688) (width 0.25) (layer "B.Cu") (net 13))
 (segment (start 85.33 58.688) (end 90.678 53.34) (width 0.25) (layer "B.Cu") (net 13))
 (segment (start 83.82 62.738) (end 93.218 53.34) (width 0.25) (layer "B.Cu") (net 17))
 (segment (start 77.216 62.738) (end 83.82 62.738) (width 0.25) (layer "B.Cu") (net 17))
 (segment (start 82.31 66.788) (end 95.758 53.34) (width 0.25) (layer "B.Cu") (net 18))
 (segment (start 77.216 66.788) (end 82.31 66.788) (width 0.25) (layer "B.Cu") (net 18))
 (segment (start 80.8 70.838) (end 98.298 53.34) (width 0.25) (layer "B.Cu") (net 19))
 (segment (start 77.216 70.838) (end 80.8 70.838) (width 0.25) (layer "B.Cu") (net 19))
 (segment (start 109.046 74.439) (end 109.571 73.914) (width 0.25) (layer "F.Cu") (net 14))
 (segment (start 97.912 74.105041) (end 98.245959 74.439) (width 0.25) (layer "F.Cu") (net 14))
 (segment (start 121.255 74.168) (end 120.984 74.439) (width 0.25) (layer "F.Cu") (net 14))
 (segment (start 109.904959 74.439) (end 109.571 74.105041) (width 0.25) (layer "F.Cu") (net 14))
 (segment (start 97.912 73.914) (end 97.912 74.105041) (width 0.25) (layer "F.Cu") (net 14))
 (segment (start 98.245959 74.439) (end 109.046 74.439) (width 0.25) (layer "F.Cu") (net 14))
 (segment (start 120.984 74.439) (end 109.904959 74.439) (width 0.25) (layer "F.Cu") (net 14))
 (segment (start 109.571 74.105041) (end 109.571 73.914) (width 0.25) (layer "F.Cu") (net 14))
 (segment (start 98.806 73.66) (end 98.552 73.914) (width 0.25) (layer "B.Cu") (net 20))
 (segment (start 93.626431 67.31) (end 97.536 67.31) (width 0.25) (layer "B.Cu") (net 20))
 (segment (start 100.838 53.34) (end 92.781 61.397) (width 0.25) (layer "B.Cu") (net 20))
 (segment (start 92.781 66.464569) (end 93.626431 67.31) (width 0.25) (layer "B.Cu") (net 20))
 (segment (start 97.536 67.31) (end 98.806 66.04) (width 0.25) (layer "B.Cu") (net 20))
 (segment (start 99.577 66.811) (end 98.806 66.04) (width 0.25) (layer "B.Cu") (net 20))
 (segment (start 92.781 61.397) (end 92.781 66.464569) (width 0.25) (layer "B.Cu") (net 20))
 (segment (start 98.806 66.04) (end 98.806 73.66) (width 0.25) (layer "B.Cu") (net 20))
 (segment (start 110.211 73.914) (end 110.236 73.889) (width 0.25) (layer "F.Cu") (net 15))
 (segment (start 110.236 73.889) (end 110.236 65.786) (width 0.25) (layer "F.Cu") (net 15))
 (segment (start 111.797999 64.224001) (end 110.236 65.786) (width 0.25) (layer "B.Cu") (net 15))
 (segment (start 110.998 53.34) (end 111.797999 54.139999) (width 0.25) (layer "B.Cu") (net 15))
 (segment (start 111.797999 54.139999) (end 111.797999 64.224001) (width 0.25) (layer "B.Cu") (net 15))
 (segment (start 121.895 67.975) (end 121.666 67.746) (width 0.25) (layer "F.Cu") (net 4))
 (segment (start 121.895 74.168) (end 121.895 67.975) (width 0.25) (layer "F.Cu") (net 4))
 (segment (start 105.918 53.34) (end 104.211 55.047) (width 0.25) (layer "B.Cu") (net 4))
 (segment (start 104.211 55.047) (end 104.211 66.365) (width 0.25) (layer "B.Cu") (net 4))
 (segment (start 104.211 66.365) (end 105.592 67.746) (width 0.25) (layer "B.Cu") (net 4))
 (segment (start 115.166 67.746) (end 121.666 67.746) (width 0.25) (layer "B.Cu") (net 4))
 (segment (start 105.592 67.746) (end 115.166 67.746) (width 0.25) (layer "B.Cu") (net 4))
 (segment (start 113.633833 53.34) (end 122.991 62.697167) (width 0.25) (layer "B.Cu") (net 8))
 (segment (start 113.538 53.34) (end 113.633833 53.34) (width 0.25) (layer "B.Cu") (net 8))
 (segment (start 150.622 72.644) (end 150.622 63.028) (width 0.25) (layer "B.Cu") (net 8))
 (segment (start 148.082 62.738) (end 146.812 64.008) (width 0.25) (layer "B.Cu") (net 8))
 (segment (start 122.991 62.697167) (end 122.991 68.635) (width 0.25) (layer "B.Cu") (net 8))
 (segment (start 150.622 63.028) (end 150.332 62.738) (width 0.25) (layer "B.Cu") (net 8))
 (segment (start 145.06 78.206) (end 150.622 72.644) (width 0.25) (layer "B.Cu") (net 8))
 (segment (start 150.332 62.738) (end 148.082 62.738) (width 0.25) (layer "B.Cu") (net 8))
 (segment (start 122.991 68.635) (end 132.562 78.206) (width 0.25) (layer "B.Cu") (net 8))
 (segment (start 132.562 78.206) (end 145.06 78.206) (width 0.25) (layer "B.Cu") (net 8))
 (segment (start 132.987 62.883) (end 134.112 64.008) (width 0.25) (layer "B.Cu") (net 10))
 (segment (start 116.078 53.34) (end 125.621 62.883) (width 0.25) (layer "B.Cu") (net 10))
 (segment (start 125.621 62.883) (end 132.987 62.883) (width 0.25) (layer "B.Cu") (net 10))
 (segment (start 135.237 63.542009) (end 135.237 70.503) (width 0.25) (layer "B.Cu") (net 11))
 (segment (start 118.618 53.34) (end 127.711 62.433) (width 0.25) (layer "B.Cu") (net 11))
 (segment (start 135.237 70.503) (end 134.112 71.628) (width 0.25) (layer "B.Cu") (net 11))
 (segment (start 127.711 62.433) (end 134.127991 62.433) (width 0.25) (layer "B.Cu") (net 11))
 (segment (start 134.127991 62.433) (end 135.237 63.542009) (width 0.25) (layer "B.Cu") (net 11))
 (segment (start 125.736 57.918) (end 138.056396 57.918) (width 0.25) (layer "B.Cu") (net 12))
 (segment (start 142.857 62.718604) (end 142.857 67.673) (width 0.25) (layer "B.Cu") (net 12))
 (segment (start 142.857 67.673) (end 146.812 71.628) (width 0.25) (layer "B.Cu") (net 12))
 (segment (start 121.158 53.34) (end 125.736 57.918) (width 0.25) (layer "B.Cu") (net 12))
 (segment (start 138.056396 57.918) (end 142.857 62.718604) (width 0.25) (layer "B.Cu") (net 12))
 (segment (start 126.408 78.656) (end 121.92 74.168) (width 0.25) (layer "B.Cu") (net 29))
 (segment (start 146.05 51.054) (end 143.764 53.34) (width 0.25) (layer "B.Cu") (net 29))
 (segment (start 149.606 51.054) (end 146.05 51.054) (width 0.25) (layer "B.Cu") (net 29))
 (segment (start 143.764 53.34) (end 152.4 61.976) (width 0.25) (layer "B.Cu") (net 29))
 (segment (start 152.4 61.976) (end 152.4 71.628) (width 0.25) (layer "B.Cu") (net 29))
 (segment (start 152.4 71.628) (end 145.372 78.656) (width 0.25) (layer "B.Cu") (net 29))
 (segment (start 145.372 78.656) (end 126.408 78.656) (width 0.25) (layer "B.Cu") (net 29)))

